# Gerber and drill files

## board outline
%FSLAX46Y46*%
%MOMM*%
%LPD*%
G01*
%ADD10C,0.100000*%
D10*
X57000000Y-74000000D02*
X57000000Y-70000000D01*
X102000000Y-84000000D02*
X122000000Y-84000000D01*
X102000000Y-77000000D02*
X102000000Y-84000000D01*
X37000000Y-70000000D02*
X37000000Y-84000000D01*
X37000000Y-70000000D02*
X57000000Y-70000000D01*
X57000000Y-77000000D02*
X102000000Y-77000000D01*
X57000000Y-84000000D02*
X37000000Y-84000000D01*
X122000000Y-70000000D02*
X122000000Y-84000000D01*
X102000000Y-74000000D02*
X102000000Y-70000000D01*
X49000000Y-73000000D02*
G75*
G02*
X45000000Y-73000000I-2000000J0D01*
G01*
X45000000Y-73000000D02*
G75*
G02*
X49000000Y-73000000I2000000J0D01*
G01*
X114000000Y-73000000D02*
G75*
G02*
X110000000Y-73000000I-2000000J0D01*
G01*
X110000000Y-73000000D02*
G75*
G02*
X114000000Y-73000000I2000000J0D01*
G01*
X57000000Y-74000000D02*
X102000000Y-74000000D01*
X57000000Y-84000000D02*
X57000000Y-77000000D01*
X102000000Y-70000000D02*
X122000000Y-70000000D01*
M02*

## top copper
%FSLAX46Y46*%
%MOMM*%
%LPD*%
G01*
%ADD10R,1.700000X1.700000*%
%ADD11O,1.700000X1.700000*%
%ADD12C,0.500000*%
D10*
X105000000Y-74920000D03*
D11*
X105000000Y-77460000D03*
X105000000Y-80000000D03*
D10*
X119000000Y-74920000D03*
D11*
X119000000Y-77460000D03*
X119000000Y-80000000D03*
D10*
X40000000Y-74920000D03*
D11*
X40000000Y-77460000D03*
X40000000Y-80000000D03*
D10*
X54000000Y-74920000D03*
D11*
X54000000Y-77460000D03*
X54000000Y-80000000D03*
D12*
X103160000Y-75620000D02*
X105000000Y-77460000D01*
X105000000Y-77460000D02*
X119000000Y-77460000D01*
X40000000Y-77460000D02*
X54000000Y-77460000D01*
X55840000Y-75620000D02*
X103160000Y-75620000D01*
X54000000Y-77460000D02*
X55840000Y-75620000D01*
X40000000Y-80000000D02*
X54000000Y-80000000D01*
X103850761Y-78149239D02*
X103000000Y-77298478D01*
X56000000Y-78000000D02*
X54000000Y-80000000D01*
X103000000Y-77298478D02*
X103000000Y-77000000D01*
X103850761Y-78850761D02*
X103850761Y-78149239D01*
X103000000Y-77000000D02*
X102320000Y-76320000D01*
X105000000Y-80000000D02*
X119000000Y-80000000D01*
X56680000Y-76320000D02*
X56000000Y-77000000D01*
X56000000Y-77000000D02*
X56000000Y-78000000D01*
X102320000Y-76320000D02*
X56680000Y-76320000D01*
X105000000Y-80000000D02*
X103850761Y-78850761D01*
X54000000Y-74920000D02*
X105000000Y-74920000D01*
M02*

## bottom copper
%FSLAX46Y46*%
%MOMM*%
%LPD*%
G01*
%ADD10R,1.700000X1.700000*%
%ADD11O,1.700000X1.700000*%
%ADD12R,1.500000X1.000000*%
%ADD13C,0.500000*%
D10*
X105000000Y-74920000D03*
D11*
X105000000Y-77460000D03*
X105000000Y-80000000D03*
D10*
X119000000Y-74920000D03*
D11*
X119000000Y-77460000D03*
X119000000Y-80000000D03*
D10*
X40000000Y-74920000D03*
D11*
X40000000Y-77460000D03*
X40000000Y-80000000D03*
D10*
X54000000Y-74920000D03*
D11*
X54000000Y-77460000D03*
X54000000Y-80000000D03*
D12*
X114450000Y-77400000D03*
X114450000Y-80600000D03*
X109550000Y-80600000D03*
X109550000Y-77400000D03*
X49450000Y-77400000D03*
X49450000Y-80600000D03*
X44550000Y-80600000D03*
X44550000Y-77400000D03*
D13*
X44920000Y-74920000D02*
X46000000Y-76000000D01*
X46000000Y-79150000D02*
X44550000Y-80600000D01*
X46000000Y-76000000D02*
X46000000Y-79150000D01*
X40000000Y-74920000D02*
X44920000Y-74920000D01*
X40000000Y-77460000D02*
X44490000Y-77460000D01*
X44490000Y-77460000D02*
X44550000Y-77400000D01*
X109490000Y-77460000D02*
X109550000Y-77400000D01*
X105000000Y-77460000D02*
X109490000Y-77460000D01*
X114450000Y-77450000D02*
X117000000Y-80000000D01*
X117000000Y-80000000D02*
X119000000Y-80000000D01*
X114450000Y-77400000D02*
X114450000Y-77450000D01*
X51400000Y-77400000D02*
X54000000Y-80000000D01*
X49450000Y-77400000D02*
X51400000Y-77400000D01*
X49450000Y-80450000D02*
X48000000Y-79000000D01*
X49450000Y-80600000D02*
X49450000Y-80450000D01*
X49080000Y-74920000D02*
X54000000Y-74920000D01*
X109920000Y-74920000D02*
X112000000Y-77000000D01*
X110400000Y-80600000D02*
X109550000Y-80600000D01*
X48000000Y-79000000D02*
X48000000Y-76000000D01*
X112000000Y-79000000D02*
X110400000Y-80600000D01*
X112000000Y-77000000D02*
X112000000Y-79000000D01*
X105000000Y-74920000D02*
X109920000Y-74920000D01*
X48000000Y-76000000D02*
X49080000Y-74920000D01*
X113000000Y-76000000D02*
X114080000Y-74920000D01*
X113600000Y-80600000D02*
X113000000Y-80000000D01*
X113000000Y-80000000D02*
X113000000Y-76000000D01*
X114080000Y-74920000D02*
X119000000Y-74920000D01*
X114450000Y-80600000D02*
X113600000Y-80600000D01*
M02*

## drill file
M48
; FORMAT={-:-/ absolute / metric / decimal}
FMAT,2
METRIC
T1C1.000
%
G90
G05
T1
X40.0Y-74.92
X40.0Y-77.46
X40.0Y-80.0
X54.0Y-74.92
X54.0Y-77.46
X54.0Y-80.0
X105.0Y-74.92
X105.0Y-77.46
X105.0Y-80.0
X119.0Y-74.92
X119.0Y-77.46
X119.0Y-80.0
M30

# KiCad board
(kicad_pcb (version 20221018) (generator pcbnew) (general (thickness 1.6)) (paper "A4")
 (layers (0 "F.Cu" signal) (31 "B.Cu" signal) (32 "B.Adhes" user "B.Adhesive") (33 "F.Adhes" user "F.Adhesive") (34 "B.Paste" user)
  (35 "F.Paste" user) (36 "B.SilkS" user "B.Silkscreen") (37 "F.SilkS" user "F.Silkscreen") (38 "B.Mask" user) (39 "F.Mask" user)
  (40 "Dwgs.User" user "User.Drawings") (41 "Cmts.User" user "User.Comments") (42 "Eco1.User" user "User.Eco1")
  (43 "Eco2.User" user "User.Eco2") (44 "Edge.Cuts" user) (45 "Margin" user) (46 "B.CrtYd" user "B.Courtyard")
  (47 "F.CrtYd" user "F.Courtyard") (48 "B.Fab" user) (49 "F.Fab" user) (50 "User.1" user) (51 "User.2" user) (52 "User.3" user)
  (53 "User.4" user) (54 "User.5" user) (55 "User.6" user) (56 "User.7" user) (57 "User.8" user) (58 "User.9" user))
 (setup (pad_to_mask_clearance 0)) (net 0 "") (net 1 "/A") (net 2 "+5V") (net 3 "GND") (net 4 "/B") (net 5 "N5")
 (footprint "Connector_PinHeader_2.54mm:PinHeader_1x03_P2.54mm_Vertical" (layer "F.Cu") (at 105 74.92)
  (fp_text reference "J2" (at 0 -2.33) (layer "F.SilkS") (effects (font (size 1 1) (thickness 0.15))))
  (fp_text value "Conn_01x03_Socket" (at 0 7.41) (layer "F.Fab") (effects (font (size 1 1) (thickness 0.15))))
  (pad "1" thru_hole rect (at 0 0) (size 1.7 1.7) (drill 1) (layers "*.Cu" "*.Mask") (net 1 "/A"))
  (pad "2" thru_hole oval (at 0 2.54) (size 1.7 1.7) (drill 1) (layers "*.Cu" "*.Mask") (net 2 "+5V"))
  (pad "3" thru_hole oval (at 0 5.08) (size 1.7 1.7) (drill 1) (layers "*.Cu" "*.Mask") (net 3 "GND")))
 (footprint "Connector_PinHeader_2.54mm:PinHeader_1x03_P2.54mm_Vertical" (layer "F.Cu") (at 119 74.92)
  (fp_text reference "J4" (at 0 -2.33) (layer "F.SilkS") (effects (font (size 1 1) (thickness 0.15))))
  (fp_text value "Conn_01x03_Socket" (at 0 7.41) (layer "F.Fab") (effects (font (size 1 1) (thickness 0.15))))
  (pad "1" thru_hole rect (at 0 0) (size 1.7 1.7) (drill 1) (layers "*.Cu" "*.Mask") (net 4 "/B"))
  (pad "2" thru_hole oval (at 0 2.54) (size 1.7 1.7) (drill 1) (layers "*.Cu" "*.Mask") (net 2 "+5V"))
  (pad "3" thru_hole oval (at 0 5.08) (size 1.7 1.7) (drill 1) (layers "*.Cu" "*.Mask") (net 3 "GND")))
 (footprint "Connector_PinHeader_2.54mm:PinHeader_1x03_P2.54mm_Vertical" (layer "F.Cu") (at 40 74.92)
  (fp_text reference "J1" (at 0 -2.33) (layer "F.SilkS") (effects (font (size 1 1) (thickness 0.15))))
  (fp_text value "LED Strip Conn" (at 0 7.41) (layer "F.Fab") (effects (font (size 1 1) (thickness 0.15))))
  (pad "1" thru_hole rect (at 0 0) (size 1.7 1.7) (drill 1) (layers "*.Cu" "*.Mask") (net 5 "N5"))
  (pad "2" thru_hole oval (at 0 2.54) (size 1.7 1.7) (drill 1) (layers "*.Cu" "*.Mask") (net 2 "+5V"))
  (pad "3" thru_hole oval (at 0 5.08) (size 1.7 1.7) (drill 1) (layers "*.Cu" "*.Mask") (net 3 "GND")))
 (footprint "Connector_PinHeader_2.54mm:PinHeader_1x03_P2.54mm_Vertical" (layer "F.Cu") (at 54 74.92)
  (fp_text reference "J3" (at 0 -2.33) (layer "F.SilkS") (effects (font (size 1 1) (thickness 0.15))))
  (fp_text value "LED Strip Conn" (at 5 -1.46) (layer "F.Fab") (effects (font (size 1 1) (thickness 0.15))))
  (pad "1" thru_hole rect (at 0 0) (size 1.7 1.7) (drill 1) (layers "*.Cu" "*.Mask") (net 1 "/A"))
  (pad "2" thru_hole oval (at 0 2.54) (size 1.7 1.7) (drill 1) (layers "*.Cu" "*.Mask") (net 2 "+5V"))
  (pad "3" thru_hole oval (at 0 5.08) (size 1.7 1.7) (drill 1) (layers "*.Cu" "*.Mask") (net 3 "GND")))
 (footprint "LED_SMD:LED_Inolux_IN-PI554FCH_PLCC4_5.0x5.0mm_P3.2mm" (layer "B.Cu") (at 112 79 180)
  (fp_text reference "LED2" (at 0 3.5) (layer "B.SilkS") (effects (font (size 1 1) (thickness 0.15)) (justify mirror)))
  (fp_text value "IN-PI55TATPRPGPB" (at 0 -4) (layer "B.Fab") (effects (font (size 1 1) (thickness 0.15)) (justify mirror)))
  (pad "1" smd rect (at -2.45 1.6 180) (size 1.5 1) (layers "B.Cu" "B.Paste" "B.Mask") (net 3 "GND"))
  (pad "2" smd rect (at -2.45 -1.6 180) (size 1.5 1) (layers "B.Cu" "B.Paste" "B.Mask") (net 4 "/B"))
  (pad "3" smd rect (at 2.45 -1.6 180) (size 1.5 1) (layers "B.Cu" "B.Paste" "B.Mask") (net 1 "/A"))
  (pad "4" smd rect (at 2.45 1.6 180) (size 1.5 1) (layers "B.Cu" "B.Paste" "B.Mask") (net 2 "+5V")))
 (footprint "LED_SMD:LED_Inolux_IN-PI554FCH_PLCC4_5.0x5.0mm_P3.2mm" (layer "B.Cu") (at 47 79 180)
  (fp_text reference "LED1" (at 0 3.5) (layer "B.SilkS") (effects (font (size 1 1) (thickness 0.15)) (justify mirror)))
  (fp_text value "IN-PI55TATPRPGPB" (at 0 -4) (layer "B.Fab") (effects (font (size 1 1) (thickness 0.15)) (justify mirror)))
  (pad "1" smd rect (at -2.45 1.6 180) (size 1.5 1) (layers "B.Cu" "B.Paste" "B.Mask") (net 3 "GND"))
  (pad "2" smd rect (at -2.45 -1.6 180) (size 1.5 1) (layers "B.Cu" "B.Paste" "B.Mask") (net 1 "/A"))
  (pad "3" smd rect (at 2.45 -1.6 180) (size 1.5 1) (layers "B.Cu" "B.Paste" "B.Mask") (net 5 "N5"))
  (pad "4" smd rect (at 2.45 1.6 180) (size 1.5 1) (layers "B.Cu" "B.Paste" "B.Mask") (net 2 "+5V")))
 (gr_line (start 57 74) (end 57 70) (stroke (width 0.1) (type default)) (layer "Edge.Cuts"))
 (gr_line (start 102 84) (end 122 84) (stroke (width 0.1) (type default)) (layer "Edge.Cuts"))
 (gr_line (start 102 77) (end 102 84) (stroke (width 0.1) (type default)) (layer "Edge.Cuts"))
 (gr_line (start 37 70) (end 37 84) (stroke (width 0.1) (type default)) (layer "Edge.Cuts"))
 (gr_line (start 37 70) (end 57 70) (stroke (width 0.1) (type default)) (layer "Edge.Cuts"))
 (gr_line (start 57 77) (end 102 77) (stroke (width 0.1) (type default)) (layer "Edge.Cuts"))
 (gr_line (start 57 84) (end 37 84) (stroke (width 0.1) (type default)) (layer "Edge.Cuts"))
 (gr_line (start 122 70) (end 122 84) (stroke (width 0.1) (type default)) (layer "Edge.Cuts"))
 (gr_line (start 102 74) (end 102 70) (stroke (width 0.1) (type default)) (layer "Edge.Cuts"))
 (gr_circle (center 47 73) (end 49 73) (stroke (width 0.1) (type default)) (fill none) (layer "Edge.Cuts"))
 (gr_circle (center 112 73) (end 110 73) (stroke (width 0.1) (type default)) (fill none) (layer "Edge.Cuts"))
 (gr_line (start 57 74) (end 102 74) (stroke (width 0.1) (type default)) (layer "Edge.Cuts"))
 (gr_line (start 57 84) (end 57 77) (stroke (width 0.1) (type default)) (layer "Edge.Cuts"))
 (gr_line (start 102 70) (end 122 70) (stroke (width 0.1) (type default)) (layer "Edge.Cuts"))
 (segment (start 44.92 74.92) (end 46 76) (width 0.5) (layer "B.Cu") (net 5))
 (segment (start 46 79.15) (end 44.55 80.6) (width 0.5) (layer "B.Cu") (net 5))
 (segment (start 46 76) (end 46 79.15) (width 0.5) (layer "B.Cu") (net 5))
 (segment (start 40 74.92) (end 44.92 74.92) (width 0.5) (layer "B.Cu") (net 5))
 (segment (start 103.16 75.62) (end 105 77.46) (width 0.5) (layer "F.Cu") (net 2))
 (segment (start 105 77.46) (end 119 77.46) (width 0.5) (layer "F.Cu") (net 2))
 (segment (start 40 77.46) (end 54 77.46) (width 0.5) (layer "F.Cu") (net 2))
 (segment (start 55.84 75.62) (end 103.16 75.62) (width 0.5) (layer "F.Cu") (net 2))
 (segment (start 54 77.46) (end 55.84 75.62) (width 0.5) (layer "F.Cu") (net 2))
 (segment (start 40 77.46) (end 44.49 77.46) (width 0.5) (layer "B.Cu") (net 2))
 (segment (start 44.49 77.46) (end 44.55 77.4) (width 0.5) (layer "B.Cu") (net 2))
 (segment (start 109.49 77.46) (end 109.55 77.4) (width 0.5) (layer "B.Cu") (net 2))
 (segment (start 105 77.46) (end 109.49 77.46) (width 0.5) (layer "B.Cu") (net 2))
 (segment (start 40 80) (end 54 80) (width 0.5) (layer "F.Cu") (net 3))
 (segment (start 103.850761 78.149239) (end 103 77.298478) (width 0.5) (layer "F.Cu") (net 3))
 (segment (start 56 78) (end 54 80) (width 0.5) (layer "F.Cu") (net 3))
 (segment (start 103 77.298478) (end 103 77) (width 0.5) (layer "F.Cu") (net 3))
 (segment (start 103.850761 78.850761) (end 103.850761 78.149239) (width 0.5) (layer "F.Cu") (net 3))
 (segment (start 103 77) (end 102.32 76.32) (width 0.5) (layer "F.Cu") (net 3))
 (segment (start 105 80) (end 119 80) (width 0.5) (layer "F.Cu") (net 3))
 (segment (start 56.68 76.32) (end 56 77) (width 0.5) (layer "F.Cu") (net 3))
 (segment (start 56 77) (end 56 78) (width 0.5) (layer "F.Cu") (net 3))
 (segment (start 102.32 76.32) (end 56.68 76.32) (width 0.5) (layer "F.Cu") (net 3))
 (segment (start 105 80) (end 103.850761 78.850761) (width 0.5) (layer "F.Cu") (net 3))
 (segment (start 114.45 77.45) (end 117 80) (width 0.5) (layer "B.Cu") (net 3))
 (segment (start 117 80) (end 119 80) (width 0.5) (layer "B.Cu") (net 3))
 (segment (start 114.45 77.4) (end 114.45 77.45) (width 0.5) (layer "B.Cu") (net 3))
 (segment (start 51.4 77.4) (end 54 80) (width 0.5) (layer "B.Cu") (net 3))
 (segment (start 49.45 77.4) (end 51.4 77.4) (width 0.5) (layer "B.Cu") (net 3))
 (segment (start 54 74.92) (end 105 74.92) (width 0.5) (layer "F.Cu") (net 1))
 (segment (start 49.45 80.45) (end 48 79) (width 0.5) (layer "B.Cu") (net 1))
 (segment (start 49.45 80.6) (end 49.45 80.45) (width 0.5) (layer "B.Cu") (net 1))
 (segment (start 49.08 74.92) (end 54 74.92) (width 0.5) (layer "B.Cu") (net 1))
 (segment (start 109.92 74.92) (end 112 77) (width 0.5) (layer "B.Cu") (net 1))
 (segment (start 110.4 80.6) (end 109.55 80.6) (width 0.5) (layer "B.Cu") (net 1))
 (segment (start 48 79) (end 48 76) (width 0.5) (layer "B.Cu") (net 1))
 (segment (start 112 79) (end 110.4 80.6) (width 0.5) (layer "B.Cu") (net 1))
 (segment (start 112 77) (end 112 79) (width 0.5) (layer "B.Cu") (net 1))
 (segment (start 105 74.92) (end 109.92 74.92) (width 0.5) (layer "B.Cu") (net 1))
 (segment (start 48 76) (end 49.08 74.92) (width 0.5) (layer "B.Cu") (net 1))
 (segment (start 113 76) (end 114.08 74.92) (width 0.5) (layer "B.Cu") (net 4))
 (segment (start 113.6 80.6) (end 113 80) (width 0.5) (layer "B.Cu") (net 4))
 (segment (start 113 80) (end 113 76) (width 0.5) (layer "B.Cu") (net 4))
 (segment (start 114.08 74.92) (end 119 74.92) (width 0.5) (layer "B.Cu") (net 4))
 (segment (start 114.45 80.6) (end 113.6 80.6) (width 0.5) (layer "B.Cu") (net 4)))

